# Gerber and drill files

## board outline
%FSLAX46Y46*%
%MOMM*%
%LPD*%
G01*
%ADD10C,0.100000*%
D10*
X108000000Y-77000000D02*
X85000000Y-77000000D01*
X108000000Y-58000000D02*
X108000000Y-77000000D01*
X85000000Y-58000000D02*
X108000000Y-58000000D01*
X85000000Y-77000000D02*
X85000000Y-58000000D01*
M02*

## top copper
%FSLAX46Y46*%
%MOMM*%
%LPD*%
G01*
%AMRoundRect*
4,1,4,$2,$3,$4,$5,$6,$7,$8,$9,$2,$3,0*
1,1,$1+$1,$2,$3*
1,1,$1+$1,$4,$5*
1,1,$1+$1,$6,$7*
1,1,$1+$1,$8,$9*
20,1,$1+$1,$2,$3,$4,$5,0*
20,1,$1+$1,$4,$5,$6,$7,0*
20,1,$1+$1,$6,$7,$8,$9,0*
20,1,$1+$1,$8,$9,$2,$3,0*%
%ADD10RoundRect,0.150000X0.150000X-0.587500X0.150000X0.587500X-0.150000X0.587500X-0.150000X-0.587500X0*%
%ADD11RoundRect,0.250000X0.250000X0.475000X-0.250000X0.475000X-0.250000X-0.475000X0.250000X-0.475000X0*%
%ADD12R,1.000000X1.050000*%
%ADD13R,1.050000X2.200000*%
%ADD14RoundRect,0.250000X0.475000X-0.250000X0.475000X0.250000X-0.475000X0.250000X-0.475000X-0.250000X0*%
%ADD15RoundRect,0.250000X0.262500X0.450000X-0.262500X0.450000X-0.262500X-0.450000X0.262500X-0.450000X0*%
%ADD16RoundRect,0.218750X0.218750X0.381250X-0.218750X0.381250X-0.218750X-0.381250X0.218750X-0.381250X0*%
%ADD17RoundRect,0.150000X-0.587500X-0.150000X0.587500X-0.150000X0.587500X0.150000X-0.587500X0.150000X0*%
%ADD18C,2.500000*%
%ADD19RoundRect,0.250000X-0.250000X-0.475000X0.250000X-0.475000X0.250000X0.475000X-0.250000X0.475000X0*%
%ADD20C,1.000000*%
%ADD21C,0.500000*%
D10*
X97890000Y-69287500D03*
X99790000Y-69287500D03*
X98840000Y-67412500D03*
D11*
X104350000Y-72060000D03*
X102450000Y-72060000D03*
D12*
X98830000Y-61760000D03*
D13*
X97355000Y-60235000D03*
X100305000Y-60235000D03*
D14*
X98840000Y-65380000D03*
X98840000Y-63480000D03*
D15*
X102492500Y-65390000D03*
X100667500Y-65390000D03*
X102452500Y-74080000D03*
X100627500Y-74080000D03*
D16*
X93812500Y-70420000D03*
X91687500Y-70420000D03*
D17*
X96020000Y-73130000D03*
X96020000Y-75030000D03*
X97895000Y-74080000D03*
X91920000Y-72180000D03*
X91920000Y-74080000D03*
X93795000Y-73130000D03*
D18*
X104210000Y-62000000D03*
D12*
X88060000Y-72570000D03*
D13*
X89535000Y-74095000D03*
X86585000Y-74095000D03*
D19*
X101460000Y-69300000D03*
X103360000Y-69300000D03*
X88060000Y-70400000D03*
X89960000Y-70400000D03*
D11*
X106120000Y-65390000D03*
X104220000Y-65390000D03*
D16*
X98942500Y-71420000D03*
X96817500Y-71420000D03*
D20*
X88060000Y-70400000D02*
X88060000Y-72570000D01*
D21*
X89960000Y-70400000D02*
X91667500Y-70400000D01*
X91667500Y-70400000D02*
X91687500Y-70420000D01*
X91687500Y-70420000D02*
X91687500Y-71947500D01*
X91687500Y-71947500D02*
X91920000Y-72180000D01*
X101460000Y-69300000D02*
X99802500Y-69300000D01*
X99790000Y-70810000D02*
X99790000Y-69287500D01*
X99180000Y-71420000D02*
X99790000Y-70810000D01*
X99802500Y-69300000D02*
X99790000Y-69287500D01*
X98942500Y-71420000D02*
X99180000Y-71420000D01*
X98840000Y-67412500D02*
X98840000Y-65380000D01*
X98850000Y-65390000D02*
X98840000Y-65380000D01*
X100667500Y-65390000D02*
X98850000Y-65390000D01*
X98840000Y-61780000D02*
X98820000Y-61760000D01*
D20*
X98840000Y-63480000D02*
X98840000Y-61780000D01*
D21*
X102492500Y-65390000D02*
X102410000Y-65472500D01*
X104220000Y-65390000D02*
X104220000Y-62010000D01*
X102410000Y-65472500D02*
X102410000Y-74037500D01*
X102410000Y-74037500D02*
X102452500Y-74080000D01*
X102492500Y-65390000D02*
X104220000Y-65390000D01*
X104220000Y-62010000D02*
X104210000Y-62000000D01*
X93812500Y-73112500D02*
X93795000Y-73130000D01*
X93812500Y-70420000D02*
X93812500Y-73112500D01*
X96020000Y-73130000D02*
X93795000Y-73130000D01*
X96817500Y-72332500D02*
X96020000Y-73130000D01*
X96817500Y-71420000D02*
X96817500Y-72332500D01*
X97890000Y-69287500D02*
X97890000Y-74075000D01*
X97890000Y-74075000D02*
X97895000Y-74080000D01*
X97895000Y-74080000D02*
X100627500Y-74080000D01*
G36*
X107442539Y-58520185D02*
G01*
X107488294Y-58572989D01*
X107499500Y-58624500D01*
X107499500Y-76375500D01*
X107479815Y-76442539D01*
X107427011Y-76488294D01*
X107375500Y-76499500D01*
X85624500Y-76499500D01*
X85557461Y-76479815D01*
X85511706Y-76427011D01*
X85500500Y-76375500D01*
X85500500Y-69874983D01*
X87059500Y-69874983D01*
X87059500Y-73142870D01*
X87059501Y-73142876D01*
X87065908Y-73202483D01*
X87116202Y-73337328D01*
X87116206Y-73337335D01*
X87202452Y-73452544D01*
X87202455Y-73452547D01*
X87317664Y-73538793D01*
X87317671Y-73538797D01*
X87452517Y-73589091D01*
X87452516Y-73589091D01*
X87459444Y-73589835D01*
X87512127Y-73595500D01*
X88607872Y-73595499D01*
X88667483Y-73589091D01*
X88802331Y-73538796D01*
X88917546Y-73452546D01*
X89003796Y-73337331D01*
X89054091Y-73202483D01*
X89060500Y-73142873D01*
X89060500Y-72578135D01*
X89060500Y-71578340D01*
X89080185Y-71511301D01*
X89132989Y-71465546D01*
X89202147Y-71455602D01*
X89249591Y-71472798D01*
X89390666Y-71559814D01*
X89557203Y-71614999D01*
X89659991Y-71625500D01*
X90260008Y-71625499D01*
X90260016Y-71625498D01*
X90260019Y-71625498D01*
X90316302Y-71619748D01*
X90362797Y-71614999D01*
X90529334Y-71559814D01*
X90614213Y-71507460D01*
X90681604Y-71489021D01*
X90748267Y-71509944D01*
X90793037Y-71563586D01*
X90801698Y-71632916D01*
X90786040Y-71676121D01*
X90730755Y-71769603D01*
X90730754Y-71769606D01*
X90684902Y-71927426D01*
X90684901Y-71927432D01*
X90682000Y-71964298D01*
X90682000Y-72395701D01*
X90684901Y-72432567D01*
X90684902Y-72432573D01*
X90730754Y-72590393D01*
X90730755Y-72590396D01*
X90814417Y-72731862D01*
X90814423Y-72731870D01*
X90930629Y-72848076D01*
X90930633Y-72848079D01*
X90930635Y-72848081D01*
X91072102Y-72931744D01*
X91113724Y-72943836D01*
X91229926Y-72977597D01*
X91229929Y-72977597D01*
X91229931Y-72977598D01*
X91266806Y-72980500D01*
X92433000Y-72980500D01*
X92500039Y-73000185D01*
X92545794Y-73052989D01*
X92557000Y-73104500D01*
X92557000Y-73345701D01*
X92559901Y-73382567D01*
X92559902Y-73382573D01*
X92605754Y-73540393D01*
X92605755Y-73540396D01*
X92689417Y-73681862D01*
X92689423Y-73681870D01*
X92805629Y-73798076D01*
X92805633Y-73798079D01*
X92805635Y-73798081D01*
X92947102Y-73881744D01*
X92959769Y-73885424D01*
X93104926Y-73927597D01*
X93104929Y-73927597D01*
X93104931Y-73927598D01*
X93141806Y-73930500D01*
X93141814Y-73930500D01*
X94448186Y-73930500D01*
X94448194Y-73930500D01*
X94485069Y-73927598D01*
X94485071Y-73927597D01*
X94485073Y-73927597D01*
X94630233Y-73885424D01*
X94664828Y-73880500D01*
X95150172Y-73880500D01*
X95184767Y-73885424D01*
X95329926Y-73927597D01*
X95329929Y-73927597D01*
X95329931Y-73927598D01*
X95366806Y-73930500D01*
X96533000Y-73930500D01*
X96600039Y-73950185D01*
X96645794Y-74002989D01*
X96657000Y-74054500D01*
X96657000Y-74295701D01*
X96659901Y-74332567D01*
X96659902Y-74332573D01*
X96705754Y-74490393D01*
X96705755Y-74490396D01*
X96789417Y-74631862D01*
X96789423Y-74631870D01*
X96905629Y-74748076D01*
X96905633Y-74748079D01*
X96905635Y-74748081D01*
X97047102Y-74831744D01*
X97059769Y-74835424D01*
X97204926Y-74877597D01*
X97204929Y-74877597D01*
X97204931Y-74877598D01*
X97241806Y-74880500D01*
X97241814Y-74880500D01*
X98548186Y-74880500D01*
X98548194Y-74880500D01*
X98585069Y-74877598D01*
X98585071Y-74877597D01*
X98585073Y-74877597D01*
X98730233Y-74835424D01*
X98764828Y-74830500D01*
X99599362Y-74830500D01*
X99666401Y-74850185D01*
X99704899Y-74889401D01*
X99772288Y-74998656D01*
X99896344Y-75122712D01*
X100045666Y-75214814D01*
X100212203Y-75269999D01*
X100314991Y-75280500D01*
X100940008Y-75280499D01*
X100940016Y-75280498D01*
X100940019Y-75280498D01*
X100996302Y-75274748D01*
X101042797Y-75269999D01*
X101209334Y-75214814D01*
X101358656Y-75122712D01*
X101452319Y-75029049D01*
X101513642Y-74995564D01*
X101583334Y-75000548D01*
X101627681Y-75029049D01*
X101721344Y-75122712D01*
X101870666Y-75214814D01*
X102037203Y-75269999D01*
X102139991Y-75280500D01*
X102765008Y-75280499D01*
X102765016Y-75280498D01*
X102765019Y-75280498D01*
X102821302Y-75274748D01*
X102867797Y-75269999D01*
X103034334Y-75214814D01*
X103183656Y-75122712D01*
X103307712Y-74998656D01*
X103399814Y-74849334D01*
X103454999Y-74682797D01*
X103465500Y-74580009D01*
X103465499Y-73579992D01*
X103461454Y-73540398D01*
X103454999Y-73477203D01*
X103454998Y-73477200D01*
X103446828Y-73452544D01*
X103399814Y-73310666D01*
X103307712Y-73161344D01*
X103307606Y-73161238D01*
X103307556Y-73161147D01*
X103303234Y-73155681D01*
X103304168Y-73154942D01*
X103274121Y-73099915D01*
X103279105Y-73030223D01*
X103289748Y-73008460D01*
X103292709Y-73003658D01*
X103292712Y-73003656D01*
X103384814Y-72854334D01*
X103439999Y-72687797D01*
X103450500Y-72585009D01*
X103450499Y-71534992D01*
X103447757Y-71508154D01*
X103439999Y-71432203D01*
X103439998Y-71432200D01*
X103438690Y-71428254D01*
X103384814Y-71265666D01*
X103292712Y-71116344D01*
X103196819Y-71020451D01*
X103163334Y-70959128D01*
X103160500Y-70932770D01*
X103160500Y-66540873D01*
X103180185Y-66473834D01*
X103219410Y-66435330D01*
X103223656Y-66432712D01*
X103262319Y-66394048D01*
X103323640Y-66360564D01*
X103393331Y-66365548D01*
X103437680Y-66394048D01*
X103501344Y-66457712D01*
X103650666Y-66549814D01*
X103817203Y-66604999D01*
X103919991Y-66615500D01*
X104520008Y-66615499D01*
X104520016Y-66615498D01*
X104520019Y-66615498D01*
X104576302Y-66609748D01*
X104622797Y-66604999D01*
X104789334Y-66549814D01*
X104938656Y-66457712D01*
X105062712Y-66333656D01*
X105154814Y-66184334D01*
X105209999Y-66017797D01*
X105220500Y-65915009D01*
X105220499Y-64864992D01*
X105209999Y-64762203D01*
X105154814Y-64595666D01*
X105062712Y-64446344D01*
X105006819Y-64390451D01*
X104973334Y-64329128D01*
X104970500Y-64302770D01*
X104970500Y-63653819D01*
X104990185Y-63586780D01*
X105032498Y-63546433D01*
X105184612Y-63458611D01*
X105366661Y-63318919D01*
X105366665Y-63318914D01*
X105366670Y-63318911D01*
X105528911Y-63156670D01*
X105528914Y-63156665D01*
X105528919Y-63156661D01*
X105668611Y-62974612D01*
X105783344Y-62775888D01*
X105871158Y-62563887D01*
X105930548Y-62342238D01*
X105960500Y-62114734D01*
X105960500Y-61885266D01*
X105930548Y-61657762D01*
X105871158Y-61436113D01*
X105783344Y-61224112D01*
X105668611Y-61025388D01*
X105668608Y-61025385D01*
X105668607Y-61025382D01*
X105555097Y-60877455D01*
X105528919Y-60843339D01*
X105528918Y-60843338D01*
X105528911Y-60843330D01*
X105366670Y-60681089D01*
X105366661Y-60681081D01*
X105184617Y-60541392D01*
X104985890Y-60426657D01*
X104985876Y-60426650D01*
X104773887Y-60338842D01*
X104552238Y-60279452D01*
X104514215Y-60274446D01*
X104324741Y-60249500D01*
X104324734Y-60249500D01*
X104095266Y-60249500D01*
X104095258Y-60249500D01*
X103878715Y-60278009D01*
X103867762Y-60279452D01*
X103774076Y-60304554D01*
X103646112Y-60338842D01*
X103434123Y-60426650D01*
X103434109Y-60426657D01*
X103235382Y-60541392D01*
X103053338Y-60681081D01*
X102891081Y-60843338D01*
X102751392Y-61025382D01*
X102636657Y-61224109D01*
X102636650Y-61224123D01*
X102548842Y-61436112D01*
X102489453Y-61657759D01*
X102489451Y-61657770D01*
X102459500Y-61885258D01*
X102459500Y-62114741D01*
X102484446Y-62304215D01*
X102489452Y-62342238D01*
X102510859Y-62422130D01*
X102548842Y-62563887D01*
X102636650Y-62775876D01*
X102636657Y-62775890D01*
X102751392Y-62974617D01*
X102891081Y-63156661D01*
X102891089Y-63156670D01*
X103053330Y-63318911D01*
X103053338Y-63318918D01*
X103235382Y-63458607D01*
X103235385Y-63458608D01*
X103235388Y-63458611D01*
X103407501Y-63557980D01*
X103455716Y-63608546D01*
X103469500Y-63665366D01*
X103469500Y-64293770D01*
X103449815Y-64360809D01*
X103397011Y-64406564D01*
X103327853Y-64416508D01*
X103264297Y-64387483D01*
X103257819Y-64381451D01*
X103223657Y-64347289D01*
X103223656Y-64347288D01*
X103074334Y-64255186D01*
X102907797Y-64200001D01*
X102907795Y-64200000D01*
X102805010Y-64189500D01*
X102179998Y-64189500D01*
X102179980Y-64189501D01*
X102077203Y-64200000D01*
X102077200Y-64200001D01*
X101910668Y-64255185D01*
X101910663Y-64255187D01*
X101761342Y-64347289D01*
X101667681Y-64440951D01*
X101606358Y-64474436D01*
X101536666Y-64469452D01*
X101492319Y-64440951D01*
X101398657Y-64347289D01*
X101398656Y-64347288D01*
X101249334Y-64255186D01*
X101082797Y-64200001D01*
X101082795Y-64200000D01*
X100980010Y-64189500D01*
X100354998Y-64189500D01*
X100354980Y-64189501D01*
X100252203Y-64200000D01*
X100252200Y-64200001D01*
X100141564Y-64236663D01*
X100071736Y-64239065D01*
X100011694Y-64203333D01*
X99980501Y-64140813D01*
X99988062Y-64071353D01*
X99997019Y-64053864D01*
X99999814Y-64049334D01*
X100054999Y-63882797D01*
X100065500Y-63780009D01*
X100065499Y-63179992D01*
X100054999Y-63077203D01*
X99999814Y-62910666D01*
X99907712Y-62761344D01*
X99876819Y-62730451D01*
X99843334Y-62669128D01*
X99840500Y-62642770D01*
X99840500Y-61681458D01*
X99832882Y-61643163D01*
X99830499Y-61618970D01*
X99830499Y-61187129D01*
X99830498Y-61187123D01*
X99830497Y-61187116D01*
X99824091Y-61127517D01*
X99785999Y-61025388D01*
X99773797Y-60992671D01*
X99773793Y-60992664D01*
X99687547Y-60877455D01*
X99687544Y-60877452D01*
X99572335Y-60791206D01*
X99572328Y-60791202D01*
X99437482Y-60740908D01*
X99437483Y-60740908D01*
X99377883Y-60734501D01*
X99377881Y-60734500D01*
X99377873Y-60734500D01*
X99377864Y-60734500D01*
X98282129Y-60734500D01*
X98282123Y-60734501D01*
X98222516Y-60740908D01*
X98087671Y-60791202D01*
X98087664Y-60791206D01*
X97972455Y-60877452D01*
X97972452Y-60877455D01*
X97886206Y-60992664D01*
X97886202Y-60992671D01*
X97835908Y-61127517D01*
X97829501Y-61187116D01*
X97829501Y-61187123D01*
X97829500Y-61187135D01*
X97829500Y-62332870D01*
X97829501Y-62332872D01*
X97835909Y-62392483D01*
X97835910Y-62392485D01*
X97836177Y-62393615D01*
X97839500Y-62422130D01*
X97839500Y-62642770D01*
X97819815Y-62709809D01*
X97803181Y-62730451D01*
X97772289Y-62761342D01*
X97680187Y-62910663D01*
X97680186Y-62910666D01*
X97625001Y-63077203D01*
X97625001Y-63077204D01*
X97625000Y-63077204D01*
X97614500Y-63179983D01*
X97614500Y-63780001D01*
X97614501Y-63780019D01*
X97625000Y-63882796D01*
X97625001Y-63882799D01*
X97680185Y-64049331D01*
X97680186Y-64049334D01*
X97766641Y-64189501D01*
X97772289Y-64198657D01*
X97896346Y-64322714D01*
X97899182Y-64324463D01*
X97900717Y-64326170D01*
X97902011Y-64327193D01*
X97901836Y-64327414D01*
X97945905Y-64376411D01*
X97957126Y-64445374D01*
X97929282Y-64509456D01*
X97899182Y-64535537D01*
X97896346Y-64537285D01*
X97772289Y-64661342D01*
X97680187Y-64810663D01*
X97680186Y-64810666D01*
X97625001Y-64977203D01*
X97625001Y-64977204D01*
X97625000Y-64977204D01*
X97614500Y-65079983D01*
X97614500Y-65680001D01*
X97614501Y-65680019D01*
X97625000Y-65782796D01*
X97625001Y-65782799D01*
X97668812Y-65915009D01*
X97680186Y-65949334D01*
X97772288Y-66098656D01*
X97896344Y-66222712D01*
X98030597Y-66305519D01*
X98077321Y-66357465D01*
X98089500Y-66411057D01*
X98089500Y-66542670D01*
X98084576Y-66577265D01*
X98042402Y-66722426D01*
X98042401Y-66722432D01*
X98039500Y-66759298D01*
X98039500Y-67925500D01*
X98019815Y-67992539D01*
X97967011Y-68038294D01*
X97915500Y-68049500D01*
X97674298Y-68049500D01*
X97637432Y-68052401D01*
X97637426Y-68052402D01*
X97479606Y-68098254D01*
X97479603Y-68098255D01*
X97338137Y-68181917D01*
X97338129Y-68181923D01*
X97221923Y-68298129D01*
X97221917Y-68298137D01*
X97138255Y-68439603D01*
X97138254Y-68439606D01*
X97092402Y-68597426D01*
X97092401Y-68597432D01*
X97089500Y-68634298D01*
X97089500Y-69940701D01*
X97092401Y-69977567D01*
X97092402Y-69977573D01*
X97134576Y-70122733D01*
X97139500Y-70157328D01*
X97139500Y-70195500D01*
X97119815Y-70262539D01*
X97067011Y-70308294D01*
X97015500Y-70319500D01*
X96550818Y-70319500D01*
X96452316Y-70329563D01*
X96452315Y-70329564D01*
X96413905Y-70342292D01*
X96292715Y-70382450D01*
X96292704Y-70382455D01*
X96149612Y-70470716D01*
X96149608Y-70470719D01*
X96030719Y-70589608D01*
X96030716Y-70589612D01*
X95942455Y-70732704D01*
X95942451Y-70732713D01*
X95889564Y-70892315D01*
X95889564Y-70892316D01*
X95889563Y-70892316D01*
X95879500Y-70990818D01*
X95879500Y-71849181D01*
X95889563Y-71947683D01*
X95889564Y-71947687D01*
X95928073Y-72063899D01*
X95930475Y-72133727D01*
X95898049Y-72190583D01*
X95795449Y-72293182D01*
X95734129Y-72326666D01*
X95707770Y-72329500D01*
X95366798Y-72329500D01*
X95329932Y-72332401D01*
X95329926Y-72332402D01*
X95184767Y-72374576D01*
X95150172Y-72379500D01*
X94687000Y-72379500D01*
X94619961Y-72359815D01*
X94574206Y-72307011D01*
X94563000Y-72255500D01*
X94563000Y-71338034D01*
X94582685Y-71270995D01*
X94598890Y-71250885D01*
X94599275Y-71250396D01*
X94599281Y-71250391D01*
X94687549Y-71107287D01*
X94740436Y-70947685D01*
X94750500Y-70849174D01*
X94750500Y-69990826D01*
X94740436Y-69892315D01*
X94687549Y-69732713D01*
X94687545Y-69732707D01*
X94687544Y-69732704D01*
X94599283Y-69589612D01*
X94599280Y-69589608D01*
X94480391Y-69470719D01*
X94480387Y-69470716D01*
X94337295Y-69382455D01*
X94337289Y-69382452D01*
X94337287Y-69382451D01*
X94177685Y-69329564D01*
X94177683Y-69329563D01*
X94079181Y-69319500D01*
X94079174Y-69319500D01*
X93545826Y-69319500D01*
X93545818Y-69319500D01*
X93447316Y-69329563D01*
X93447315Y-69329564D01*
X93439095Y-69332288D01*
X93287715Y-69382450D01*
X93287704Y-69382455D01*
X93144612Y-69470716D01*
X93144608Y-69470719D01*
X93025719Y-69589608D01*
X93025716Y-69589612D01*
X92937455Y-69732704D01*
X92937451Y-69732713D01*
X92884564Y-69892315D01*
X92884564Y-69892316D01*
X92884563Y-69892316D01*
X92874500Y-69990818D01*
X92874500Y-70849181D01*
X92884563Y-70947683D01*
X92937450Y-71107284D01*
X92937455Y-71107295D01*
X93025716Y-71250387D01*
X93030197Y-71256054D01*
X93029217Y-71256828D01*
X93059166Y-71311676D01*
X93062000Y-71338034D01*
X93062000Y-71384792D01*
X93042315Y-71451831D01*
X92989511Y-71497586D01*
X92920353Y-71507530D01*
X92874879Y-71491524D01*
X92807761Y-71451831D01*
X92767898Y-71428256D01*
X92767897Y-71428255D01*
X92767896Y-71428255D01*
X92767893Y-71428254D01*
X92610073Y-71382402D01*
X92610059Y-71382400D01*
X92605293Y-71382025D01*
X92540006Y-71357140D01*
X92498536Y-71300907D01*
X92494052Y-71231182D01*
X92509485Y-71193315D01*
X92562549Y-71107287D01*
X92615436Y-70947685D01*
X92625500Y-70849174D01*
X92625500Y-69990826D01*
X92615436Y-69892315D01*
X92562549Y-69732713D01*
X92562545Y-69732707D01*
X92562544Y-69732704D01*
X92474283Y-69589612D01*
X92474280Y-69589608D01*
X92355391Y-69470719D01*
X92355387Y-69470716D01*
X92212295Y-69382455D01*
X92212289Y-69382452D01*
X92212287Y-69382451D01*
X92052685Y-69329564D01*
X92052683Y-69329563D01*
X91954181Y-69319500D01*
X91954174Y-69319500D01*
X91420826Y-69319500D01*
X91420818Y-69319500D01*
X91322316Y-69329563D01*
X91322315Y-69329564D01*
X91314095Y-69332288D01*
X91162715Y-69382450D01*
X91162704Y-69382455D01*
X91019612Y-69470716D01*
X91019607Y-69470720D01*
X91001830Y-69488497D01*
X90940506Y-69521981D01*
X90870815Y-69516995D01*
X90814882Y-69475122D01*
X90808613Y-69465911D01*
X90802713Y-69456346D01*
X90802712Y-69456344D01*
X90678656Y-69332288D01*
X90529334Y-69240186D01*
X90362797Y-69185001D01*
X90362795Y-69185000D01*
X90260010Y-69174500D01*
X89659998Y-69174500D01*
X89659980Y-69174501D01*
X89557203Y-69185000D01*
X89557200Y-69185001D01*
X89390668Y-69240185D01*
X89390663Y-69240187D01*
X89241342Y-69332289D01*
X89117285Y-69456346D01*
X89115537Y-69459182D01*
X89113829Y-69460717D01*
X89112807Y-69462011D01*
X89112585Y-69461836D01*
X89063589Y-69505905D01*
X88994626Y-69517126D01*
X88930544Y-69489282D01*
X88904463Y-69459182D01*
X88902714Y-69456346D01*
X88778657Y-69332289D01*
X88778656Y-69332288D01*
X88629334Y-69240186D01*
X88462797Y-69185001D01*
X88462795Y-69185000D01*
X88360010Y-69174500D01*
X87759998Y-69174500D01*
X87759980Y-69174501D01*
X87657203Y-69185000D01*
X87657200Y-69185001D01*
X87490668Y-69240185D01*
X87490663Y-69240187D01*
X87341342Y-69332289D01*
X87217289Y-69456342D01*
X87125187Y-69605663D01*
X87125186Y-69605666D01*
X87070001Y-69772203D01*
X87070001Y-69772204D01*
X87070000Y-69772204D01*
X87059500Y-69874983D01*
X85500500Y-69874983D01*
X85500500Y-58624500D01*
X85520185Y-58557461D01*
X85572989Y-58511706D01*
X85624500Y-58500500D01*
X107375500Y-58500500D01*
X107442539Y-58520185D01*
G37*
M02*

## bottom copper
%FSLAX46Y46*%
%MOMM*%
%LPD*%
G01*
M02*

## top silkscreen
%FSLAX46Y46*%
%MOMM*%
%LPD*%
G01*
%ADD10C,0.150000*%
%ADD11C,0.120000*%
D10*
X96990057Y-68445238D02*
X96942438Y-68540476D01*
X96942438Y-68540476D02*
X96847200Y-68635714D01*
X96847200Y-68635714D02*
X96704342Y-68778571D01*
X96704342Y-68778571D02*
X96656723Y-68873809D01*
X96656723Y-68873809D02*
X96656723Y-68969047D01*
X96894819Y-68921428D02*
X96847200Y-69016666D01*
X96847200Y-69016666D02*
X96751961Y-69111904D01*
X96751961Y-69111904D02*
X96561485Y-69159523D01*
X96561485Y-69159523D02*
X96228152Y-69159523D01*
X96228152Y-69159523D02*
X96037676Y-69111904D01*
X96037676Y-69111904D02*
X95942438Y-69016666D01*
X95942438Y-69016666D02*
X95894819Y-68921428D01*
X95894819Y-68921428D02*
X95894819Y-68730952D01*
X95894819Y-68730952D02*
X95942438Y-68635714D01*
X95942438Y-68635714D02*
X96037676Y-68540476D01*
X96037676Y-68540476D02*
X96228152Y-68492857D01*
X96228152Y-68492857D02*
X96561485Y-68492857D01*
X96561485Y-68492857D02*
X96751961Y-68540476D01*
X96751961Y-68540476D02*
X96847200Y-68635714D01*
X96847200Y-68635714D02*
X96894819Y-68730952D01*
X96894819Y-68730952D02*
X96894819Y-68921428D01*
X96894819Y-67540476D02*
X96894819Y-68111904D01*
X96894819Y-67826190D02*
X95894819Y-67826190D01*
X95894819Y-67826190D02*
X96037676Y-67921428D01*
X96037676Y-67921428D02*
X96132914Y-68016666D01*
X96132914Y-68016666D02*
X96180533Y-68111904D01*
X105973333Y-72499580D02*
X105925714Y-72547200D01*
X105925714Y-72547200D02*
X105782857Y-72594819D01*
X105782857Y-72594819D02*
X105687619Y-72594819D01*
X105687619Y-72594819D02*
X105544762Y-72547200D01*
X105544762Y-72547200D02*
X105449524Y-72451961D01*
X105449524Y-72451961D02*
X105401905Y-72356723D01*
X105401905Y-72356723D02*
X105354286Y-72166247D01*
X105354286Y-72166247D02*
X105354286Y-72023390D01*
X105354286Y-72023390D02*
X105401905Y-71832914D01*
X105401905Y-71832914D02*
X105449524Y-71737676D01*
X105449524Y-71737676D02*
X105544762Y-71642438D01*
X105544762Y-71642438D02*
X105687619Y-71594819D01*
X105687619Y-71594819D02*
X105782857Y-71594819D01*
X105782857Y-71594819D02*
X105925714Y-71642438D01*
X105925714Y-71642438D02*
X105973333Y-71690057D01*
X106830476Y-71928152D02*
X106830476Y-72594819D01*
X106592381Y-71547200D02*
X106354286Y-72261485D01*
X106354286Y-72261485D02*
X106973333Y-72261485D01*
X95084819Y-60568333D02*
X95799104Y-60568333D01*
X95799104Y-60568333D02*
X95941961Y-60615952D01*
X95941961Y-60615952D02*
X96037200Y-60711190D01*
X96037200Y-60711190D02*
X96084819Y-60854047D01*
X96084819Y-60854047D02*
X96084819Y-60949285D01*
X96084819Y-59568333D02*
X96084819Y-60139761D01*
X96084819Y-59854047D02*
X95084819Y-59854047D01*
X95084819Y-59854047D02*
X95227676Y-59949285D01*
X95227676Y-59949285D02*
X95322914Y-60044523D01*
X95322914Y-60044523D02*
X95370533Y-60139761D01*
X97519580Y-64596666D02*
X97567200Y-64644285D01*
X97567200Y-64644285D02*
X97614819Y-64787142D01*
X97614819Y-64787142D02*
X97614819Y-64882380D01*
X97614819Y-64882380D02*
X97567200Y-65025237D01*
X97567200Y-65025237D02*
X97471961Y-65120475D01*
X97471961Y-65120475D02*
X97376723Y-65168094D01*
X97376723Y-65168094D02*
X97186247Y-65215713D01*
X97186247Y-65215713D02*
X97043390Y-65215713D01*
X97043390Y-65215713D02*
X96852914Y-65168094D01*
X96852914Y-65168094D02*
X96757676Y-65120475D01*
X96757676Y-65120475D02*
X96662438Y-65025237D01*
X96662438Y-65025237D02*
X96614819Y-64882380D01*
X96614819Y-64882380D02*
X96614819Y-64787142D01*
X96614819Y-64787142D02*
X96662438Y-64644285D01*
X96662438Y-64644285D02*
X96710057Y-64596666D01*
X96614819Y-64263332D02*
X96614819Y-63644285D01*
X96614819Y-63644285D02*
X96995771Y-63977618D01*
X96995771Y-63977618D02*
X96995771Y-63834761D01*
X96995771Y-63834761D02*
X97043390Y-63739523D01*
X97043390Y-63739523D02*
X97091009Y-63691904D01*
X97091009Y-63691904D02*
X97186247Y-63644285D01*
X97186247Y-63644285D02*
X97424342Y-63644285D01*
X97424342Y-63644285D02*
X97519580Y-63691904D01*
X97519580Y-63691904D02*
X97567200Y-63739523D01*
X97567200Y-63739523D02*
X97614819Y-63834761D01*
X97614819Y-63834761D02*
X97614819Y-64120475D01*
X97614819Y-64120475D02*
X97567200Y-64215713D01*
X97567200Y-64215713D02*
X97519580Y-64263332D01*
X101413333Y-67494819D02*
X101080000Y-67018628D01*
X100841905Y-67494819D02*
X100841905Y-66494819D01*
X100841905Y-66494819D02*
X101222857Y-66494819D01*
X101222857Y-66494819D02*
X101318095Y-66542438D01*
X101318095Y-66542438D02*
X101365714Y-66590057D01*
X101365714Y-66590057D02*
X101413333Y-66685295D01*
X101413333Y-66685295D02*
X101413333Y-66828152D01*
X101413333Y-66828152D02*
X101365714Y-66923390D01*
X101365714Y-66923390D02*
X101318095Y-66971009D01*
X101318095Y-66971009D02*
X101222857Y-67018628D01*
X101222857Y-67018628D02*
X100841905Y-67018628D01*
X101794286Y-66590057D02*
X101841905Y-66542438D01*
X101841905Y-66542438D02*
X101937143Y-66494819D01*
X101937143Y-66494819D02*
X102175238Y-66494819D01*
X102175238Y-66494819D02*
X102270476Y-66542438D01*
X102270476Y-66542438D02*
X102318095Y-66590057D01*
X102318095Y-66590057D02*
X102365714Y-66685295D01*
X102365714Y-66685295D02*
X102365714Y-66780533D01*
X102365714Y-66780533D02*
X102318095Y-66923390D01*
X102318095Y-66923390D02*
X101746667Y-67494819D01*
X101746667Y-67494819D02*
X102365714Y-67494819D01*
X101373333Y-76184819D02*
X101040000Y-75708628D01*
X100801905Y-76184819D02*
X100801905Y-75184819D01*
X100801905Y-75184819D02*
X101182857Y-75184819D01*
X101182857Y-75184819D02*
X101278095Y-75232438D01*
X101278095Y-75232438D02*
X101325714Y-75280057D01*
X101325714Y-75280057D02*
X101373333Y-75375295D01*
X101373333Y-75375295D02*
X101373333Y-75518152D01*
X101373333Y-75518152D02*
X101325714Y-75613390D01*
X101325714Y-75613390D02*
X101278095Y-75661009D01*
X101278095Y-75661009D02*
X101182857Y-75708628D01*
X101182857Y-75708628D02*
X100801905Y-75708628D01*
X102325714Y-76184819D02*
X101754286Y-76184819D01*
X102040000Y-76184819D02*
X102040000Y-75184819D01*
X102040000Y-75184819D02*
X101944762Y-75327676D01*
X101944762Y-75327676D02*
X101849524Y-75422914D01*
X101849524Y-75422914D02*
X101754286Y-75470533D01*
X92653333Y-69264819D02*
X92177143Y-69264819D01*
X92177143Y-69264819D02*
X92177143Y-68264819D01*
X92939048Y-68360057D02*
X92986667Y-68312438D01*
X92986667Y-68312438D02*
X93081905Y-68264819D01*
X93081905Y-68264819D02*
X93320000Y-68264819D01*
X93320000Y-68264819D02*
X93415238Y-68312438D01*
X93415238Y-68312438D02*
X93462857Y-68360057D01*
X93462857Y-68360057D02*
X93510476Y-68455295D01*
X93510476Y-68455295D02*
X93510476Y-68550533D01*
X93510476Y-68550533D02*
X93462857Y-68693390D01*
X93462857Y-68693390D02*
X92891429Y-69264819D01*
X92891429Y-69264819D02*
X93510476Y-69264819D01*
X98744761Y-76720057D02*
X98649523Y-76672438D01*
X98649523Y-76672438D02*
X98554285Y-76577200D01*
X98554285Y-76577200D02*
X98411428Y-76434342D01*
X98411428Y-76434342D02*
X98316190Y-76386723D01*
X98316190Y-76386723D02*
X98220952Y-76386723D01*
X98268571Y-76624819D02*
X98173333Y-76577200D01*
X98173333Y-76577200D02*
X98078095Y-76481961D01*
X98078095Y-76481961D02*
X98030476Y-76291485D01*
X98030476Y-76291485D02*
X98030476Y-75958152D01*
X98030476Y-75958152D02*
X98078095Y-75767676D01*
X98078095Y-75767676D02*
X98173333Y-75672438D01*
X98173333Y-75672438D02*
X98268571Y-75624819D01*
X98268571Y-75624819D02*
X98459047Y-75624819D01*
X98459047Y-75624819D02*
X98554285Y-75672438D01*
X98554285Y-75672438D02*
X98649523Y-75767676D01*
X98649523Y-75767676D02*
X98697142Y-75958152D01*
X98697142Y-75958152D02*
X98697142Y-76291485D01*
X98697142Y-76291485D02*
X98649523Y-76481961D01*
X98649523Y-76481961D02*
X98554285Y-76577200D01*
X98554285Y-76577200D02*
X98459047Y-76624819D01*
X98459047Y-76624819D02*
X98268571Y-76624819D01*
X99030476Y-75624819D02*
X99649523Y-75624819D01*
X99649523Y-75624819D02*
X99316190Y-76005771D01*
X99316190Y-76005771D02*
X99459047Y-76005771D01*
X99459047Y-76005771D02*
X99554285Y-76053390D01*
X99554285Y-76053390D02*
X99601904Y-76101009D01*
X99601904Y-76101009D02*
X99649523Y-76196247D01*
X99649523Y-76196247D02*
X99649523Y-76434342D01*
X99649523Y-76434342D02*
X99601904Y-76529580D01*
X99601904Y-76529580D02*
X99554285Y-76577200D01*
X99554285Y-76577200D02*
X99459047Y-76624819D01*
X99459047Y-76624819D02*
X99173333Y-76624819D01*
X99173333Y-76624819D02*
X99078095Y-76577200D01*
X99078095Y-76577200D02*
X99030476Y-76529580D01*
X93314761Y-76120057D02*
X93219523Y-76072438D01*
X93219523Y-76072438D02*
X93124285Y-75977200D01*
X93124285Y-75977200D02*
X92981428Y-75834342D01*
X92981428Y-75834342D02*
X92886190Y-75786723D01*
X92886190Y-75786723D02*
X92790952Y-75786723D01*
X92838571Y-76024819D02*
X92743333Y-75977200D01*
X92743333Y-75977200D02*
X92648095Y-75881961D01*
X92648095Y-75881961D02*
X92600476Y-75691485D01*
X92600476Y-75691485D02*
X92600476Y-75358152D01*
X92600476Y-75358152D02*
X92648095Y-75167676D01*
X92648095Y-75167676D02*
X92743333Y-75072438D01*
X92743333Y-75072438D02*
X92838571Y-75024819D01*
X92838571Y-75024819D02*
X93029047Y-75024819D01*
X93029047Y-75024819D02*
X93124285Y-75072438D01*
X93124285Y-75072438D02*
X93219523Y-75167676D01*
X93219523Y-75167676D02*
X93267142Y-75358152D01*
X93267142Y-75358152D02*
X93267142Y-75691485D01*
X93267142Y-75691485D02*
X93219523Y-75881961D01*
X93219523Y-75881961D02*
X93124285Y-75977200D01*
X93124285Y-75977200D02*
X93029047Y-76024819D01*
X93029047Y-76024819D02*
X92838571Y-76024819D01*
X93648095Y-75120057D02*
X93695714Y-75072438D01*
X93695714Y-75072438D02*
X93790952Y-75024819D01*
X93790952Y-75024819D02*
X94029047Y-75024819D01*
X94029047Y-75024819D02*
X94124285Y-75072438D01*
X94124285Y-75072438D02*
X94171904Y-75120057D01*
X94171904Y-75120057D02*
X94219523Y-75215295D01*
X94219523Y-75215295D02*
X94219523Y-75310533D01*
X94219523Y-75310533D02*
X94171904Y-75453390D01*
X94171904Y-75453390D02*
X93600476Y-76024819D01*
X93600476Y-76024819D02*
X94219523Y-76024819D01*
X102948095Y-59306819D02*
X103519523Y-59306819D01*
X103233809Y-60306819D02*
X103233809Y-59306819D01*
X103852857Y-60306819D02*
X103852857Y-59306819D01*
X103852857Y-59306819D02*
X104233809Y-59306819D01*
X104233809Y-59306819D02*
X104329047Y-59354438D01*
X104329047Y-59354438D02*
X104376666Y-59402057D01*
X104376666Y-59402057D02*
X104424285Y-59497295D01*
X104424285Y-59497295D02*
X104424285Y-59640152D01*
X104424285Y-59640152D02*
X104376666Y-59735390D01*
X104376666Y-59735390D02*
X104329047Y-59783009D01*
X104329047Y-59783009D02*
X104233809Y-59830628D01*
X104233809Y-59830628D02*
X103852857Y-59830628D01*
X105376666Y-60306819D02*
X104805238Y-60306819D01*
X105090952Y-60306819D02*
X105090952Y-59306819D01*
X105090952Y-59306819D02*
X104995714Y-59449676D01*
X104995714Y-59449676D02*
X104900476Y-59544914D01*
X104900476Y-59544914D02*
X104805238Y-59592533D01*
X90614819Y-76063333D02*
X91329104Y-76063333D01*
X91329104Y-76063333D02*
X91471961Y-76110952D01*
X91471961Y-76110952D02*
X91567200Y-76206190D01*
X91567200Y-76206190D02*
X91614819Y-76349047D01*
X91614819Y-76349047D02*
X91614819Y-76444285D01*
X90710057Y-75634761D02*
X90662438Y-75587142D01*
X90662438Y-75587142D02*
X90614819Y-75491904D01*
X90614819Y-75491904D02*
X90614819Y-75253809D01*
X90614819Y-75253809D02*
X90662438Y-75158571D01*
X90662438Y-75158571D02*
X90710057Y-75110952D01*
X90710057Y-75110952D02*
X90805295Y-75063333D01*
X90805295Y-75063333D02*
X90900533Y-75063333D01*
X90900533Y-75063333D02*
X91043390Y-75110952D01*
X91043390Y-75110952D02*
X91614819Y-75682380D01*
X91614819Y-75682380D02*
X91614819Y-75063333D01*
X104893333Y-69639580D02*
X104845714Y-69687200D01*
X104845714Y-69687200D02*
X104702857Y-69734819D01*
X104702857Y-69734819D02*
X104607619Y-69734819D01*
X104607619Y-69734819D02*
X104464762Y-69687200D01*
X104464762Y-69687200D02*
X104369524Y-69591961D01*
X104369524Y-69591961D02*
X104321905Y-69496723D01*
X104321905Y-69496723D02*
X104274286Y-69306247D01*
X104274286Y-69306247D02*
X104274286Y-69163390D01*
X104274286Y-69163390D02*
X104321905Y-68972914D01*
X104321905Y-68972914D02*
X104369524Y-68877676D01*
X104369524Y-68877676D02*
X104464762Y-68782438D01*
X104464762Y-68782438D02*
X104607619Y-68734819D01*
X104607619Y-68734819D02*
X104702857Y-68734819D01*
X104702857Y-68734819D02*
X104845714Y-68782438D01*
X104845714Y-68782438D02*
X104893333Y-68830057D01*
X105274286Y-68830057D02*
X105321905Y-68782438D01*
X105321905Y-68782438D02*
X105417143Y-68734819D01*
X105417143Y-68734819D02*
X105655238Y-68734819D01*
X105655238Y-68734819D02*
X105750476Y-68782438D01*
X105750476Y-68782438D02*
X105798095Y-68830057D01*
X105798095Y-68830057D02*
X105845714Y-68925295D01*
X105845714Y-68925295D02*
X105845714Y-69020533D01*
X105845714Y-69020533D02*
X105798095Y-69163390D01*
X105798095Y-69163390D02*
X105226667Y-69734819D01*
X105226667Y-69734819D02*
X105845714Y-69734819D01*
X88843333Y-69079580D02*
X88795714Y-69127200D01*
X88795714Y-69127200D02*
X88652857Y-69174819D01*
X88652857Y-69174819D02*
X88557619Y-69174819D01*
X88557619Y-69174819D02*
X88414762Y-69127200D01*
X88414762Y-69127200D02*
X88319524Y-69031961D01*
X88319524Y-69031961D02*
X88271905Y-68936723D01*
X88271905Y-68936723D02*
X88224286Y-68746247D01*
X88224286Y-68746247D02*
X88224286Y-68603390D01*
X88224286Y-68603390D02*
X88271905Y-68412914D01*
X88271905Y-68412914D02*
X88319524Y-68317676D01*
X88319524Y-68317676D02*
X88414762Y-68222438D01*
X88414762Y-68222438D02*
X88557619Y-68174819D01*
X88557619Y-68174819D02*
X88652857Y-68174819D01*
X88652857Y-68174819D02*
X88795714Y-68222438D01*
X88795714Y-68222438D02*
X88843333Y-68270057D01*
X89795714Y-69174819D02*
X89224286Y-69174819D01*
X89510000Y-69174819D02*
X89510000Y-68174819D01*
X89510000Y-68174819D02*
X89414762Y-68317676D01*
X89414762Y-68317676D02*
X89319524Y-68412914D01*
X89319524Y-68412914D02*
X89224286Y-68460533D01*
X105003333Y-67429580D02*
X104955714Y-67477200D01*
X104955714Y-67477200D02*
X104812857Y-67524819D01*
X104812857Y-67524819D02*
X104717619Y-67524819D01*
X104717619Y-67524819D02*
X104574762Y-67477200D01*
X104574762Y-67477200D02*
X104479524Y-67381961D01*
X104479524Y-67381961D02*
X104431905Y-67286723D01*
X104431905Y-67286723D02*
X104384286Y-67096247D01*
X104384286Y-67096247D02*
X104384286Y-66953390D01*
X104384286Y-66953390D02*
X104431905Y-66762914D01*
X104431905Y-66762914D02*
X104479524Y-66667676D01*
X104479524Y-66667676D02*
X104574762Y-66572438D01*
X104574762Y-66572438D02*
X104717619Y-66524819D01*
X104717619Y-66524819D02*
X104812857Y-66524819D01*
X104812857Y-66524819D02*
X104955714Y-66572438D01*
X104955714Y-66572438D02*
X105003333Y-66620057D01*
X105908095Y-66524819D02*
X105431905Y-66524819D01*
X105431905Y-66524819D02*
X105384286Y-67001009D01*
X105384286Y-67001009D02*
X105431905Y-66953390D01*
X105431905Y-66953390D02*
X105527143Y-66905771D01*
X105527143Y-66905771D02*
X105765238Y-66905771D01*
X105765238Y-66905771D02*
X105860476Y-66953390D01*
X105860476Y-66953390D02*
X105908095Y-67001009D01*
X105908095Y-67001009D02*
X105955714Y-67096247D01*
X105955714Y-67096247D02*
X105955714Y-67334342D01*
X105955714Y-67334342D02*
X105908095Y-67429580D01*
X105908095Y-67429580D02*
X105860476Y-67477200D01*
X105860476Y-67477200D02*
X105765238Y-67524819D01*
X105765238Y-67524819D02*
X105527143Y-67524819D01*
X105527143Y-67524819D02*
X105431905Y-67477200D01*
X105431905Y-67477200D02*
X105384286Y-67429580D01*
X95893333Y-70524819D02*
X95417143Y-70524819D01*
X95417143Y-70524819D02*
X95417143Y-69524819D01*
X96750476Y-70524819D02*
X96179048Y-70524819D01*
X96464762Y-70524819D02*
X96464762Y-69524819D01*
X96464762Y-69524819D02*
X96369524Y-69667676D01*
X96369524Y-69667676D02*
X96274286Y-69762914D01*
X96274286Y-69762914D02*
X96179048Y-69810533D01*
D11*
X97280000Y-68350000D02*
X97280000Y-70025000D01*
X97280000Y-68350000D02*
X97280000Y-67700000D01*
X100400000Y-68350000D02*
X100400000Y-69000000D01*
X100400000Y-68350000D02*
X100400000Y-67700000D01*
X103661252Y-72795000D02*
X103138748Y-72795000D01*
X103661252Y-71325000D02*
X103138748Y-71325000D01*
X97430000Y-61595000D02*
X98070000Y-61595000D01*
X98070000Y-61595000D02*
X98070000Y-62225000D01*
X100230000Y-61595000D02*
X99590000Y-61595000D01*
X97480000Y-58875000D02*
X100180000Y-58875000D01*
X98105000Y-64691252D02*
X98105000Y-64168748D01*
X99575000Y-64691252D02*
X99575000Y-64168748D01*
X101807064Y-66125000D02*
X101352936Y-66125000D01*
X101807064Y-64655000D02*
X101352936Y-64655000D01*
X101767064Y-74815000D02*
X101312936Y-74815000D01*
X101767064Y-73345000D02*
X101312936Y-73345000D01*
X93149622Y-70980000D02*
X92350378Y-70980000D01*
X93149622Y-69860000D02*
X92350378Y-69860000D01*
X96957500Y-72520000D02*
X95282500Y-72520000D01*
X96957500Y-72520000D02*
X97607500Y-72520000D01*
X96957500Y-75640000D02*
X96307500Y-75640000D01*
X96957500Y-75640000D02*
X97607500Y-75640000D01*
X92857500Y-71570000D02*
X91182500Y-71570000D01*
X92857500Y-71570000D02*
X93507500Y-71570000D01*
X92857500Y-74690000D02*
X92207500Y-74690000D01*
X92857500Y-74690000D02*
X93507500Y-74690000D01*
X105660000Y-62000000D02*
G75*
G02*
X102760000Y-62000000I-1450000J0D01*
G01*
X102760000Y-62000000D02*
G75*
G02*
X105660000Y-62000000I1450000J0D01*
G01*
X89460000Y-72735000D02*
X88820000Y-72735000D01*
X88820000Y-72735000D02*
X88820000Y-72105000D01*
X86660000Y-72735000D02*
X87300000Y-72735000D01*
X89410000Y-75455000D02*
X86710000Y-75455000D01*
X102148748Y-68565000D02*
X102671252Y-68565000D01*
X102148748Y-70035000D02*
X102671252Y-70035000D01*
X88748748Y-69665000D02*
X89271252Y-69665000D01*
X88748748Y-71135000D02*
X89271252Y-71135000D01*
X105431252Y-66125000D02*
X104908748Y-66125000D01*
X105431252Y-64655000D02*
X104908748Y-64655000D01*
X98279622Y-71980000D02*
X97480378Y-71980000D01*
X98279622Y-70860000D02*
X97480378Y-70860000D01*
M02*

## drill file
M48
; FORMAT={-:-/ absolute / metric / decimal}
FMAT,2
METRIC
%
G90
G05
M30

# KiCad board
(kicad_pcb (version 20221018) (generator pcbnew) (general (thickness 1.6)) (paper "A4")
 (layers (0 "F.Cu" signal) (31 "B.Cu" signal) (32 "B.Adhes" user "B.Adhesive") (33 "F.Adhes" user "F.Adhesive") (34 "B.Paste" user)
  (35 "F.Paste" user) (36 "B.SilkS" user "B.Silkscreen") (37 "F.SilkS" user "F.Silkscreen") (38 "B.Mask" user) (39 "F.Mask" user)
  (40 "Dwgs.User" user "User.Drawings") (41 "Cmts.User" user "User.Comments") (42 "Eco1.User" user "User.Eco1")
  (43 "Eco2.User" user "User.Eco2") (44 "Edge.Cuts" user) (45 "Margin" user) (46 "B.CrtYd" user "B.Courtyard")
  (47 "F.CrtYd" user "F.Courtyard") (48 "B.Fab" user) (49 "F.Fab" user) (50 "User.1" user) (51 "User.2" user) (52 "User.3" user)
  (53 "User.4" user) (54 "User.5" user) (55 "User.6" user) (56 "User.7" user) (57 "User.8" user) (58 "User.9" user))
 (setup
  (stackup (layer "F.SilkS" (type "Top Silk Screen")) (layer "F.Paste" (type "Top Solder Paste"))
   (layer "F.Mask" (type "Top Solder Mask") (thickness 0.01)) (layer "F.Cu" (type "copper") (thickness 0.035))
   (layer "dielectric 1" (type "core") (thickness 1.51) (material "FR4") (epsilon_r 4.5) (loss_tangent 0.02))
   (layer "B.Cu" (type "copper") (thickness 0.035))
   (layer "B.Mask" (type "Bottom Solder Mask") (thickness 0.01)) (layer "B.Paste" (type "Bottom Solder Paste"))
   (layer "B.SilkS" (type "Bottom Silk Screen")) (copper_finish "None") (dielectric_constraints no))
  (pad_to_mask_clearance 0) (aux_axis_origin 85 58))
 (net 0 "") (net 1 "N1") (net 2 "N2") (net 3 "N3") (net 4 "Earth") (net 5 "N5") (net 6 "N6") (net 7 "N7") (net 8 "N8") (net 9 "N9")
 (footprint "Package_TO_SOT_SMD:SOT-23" (layer "F.Cu") (at 98.84 68.35 90)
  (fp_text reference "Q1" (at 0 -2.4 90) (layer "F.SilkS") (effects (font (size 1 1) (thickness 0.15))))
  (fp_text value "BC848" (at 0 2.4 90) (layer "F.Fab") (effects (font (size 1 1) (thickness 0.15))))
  (fp_line (start 0 -1.56) (end -1.675 -1.56) (stroke (width 0.12) (type solid)) (layer "F.SilkS"))
  (fp_line (start 0 -1.56) (end 0.65 -1.56) (stroke (width 0.12) (type solid)) (layer "F.SilkS"))
  (fp_line (start 0 1.56) (end -0.65 1.56) (stroke (width 0.12) (type solid)) (layer "F.SilkS"))
  (fp_line (start 0 1.56) (end 0.65 1.56) (stroke (width 0.12) (type solid)) (layer "F.SilkS"))
  (pad "1" smd roundrect (at -0.9375 -0.95 90) (size 1.475 0.6) (layers "F.Cu" "F.Paste" "F.Mask") (roundrect_rratio 0.25) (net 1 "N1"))
  (pad "2" smd roundrect (at -0.9375 0.95 90) (size 1.475 0.6) (layers "F.Cu" "F.Paste" "F.Mask") (roundrect_rratio 0.25) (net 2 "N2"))
  (pad "3" smd roundrect (at 0.9375 0 90) (size 1.475 0.6) (layers "F.Cu" "F.Paste" "F.Mask") (roundrect_rratio 0.25) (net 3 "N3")))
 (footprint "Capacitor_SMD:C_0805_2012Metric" (layer "F.Cu") (at 103.4 72.06 180)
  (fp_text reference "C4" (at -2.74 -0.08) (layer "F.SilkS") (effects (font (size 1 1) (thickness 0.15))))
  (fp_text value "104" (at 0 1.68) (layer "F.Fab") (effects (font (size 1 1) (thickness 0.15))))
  (fp_line (start -0.261252 -0.735) (end 0.261252 -0.735) (stroke (width 0.12) (type solid)) (layer "F.SilkS"))
  (fp_line (start -0.261252 0.735) (end 0.261252 0.735) (stroke (width 0.12) (type solid)) (layer "F.SilkS"))
  (pad "1" smd roundrect (at -0.95 0 180) (size 1 1.45) (layers "F.Cu" "F.Paste" "F.Mask") (roundrect_rratio 0.25) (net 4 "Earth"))
  (pad "2" smd roundrect (at 0.95 0 180) (size 1 1.45) (layers "F.Cu" "F.Paste" "F.Mask") (roundrect_rratio 0.25) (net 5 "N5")))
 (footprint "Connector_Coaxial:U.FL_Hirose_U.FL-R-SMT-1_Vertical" (layer "F.Cu") (at 98.83 60.71 90)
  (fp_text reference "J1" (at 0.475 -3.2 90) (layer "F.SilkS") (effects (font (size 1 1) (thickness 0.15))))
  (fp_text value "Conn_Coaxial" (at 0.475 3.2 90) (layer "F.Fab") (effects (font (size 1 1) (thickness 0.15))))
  (fp_line (start -0.885 -1.4) (end -0.885 -0.76) (stroke (width 0.12) (type solid)) (layer "F.SilkS"))
  (fp_line (start -0.885 -0.76) (end -1.515 -0.76) (stroke (width 0.12) (type solid)) (layer "F.SilkS"))
  (fp_line (start -0.885 1.4) (end -0.885 0.76) (stroke (width 0.12) (type solid)) (layer "F.SilkS"))
  (fp_line (start 1.835 -1.35) (end 1.835 1.35) (stroke (width 0.12) (type solid)) (layer "F.SilkS"))
  (pad "1" smd rect (at -1.05 0 90) (size 1.05 1) (layers "F.Cu" "F.Paste" "F.Mask") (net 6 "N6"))
  (pad "2" smd rect (at 0.475 -1.475 90) (size 2.2 1.05) (layers "F.Cu" "F.Paste" "F.Mask") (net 4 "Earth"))
  (pad "2" smd rect (at 0.475 1.475 90) (size 2.2 1.05) (layers "F.Cu" "F.Paste" "F.Mask") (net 4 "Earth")))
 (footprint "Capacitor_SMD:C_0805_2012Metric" (layer "F.Cu") (at 98.84 64.43 90)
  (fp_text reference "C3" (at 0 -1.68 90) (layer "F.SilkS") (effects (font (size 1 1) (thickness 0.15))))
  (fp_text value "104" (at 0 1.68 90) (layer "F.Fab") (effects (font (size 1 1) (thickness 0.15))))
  (fp_line (start -0.261252 -0.735) (end 0.261252 -0.735) (stroke (width 0.12) (type solid)) (layer "F.SilkS"))
  (fp_line (start -0.261252 0.735) (end 0.261252 0.735) (stroke (width 0.12) (type solid)) (layer "F.SilkS"))
  (pad "1" smd roundrect (at -0.95 0 90) (size 1 1.45) (layers "F.Cu" "F.Paste" "F.Mask") (roundrect_rratio 0.25) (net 3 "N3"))
  (pad "2" smd roundrect (at 0.95 0 90) (size 1 1.45) (layers "F.Cu" "F.Paste" "F.Mask") (roundrect_rratio 0.25) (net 6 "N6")))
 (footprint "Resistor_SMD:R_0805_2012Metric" (layer "F.Cu") (at 101.58 65.39 180)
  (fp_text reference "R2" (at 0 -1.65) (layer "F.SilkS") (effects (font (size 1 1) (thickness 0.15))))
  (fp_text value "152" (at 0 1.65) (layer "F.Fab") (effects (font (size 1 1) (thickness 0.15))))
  (fp_line (start -0.227064 -0.735) (end 0.227064 -0.735) (stroke (width 0.12) (type solid)) (layer "F.SilkS"))
  (fp_line (start -0.227064 0.735) (end 0.227064 0.735) (stroke (width 0.12) (type solid)) (layer "F.SilkS"))
  (pad "1" smd roundrect (at -0.9125 0 180) (size 1.025 1.4) (layers "F.Cu" "F.Paste" "F.Mask") (roundrect_rratio 0.243902439) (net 5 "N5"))
  (pad "2" smd roundrect (at 0.9125 0 180) (size 1.025 1.4) (layers "F.Cu" "F.Paste" "F.Mask") (roundrect_rratio 0.243902439) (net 3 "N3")))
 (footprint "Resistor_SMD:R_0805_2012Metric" (layer "F.Cu") (at 101.54 74.08 180)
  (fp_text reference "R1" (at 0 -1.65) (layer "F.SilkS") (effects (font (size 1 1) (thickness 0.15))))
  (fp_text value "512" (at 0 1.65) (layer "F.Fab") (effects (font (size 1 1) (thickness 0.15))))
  (fp_line (start -0.227064 -0.735) (end 0.227064 -0.735) (stroke (width 0.12) (type solid)) (layer "F.SilkS"))
  (fp_line (start -0.227064 0.735) (end 0.227064 0.735) (stroke (width 0.12) (type solid)) (layer "F.SilkS"))
  (pad "1" smd roundrect (at -0.9125 0 180) (size 1.025 1.4) (layers "F.Cu" "F.Paste" "F.Mask") (roundrect_rratio 0.243902439) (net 5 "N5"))
  (pad "2" smd roundrect (at 0.9125 0 180) (size 1.025 1.4) (layers "F.Cu" "F.Paste" "F.Mask") (roundrect_rratio 0.243902439) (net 1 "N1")))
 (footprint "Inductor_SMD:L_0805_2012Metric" (layer "F.Cu") (at 92.75 70.42 180)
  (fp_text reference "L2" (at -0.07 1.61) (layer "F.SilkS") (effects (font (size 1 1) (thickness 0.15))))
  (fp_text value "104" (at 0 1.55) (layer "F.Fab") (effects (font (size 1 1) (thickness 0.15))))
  (fp_line (start -0.399622 -0.56) (end 0.399622 -0.56) (stroke (width 0.12) (type solid)) (layer "F.SilkS"))
  (fp_line (start -0.399622 0.56) (end 0.399622 0.56) (stroke (width 0.12) (type solid)) (layer "F.SilkS"))
  (pad "1" smd roundrect (at -1.0625 0 180) (size 0.875 1.2) (layers "F.Cu" "F.Paste" "F.Mask") (roundrect_rratio 0.25) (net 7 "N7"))
  (pad "2" smd roundrect (at 1.0625 0 180) (size 0.875 1.2) (layers "F.Cu" "F.Paste" "F.Mask") (roundrect_rratio 0.25) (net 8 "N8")))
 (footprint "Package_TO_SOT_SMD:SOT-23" (layer "F.Cu") (at 96.9575 74.08)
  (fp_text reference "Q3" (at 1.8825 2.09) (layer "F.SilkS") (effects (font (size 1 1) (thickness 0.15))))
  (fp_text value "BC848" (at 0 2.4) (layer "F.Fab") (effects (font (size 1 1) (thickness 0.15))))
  (fp_line (start 0 -1.56) (end -1.675 -1.56) (stroke (width 0.12) (type solid)) (layer "F.SilkS"))
  (fp_line (start 0 -1.56) (end 0.65 -1.56) (stroke (width 0.12) (type solid)) (layer "F.SilkS"))
  (fp_line (start 0 1.56) (end -0.65 1.56) (stroke (width 0.12) (type solid)) (layer "F.SilkS"))
  (fp_line (start 0 1.56) (end 0.65 1.56) (stroke (width 0.12) (type solid)) (layer "F.SilkS"))
  (pad "1" smd roundrect (at -0.9375 -0.95) (size 1.475 0.6) (layers "F.Cu" "F.Paste" "F.Mask") (roundrect_rratio 0.25) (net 7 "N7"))
  (pad "2" smd roundrect (at -0.9375 0.95) (size 1.475 0.6) (layers "F.Cu" "F.Paste" "F.Mask") (roundrect_rratio 0.25) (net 4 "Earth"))
  (pad "3" smd roundrect (at 0.9375 0) (size 1.475 0.6) (layers "F.Cu" "F.Paste" "F.Mask") (roundrect_rratio 0.25) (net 1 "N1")))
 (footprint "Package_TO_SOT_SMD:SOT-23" (layer "F.Cu") (at 92.8575 73.13)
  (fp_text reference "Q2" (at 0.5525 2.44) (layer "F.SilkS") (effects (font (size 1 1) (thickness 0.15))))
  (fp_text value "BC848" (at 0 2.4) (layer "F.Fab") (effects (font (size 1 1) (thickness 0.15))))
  (fp_line (start 0 -1.56) (end -1.675 -1.56) (stroke (width 0.12) (type solid)) (layer "F.SilkS"))
  (fp_line (start 0 -1.56) (end 0.65 -1.56) (stroke (width 0.12) (type solid)) (layer "F.SilkS"))
  (fp_line (start 0 1.56) (end -0.65 1.56) (stroke (width 0.12) (type solid)) (layer "F.SilkS"))
  (fp_line (start 0 1.56) (end 0.65 1.56) (stroke (width 0.12) (type solid)) (layer "F.SilkS"))
  (pad "1" smd roundrect (at -0.9375 -0.95) (size 1.475 0.6) (layers "F.Cu" "F.Paste" "F.Mask") (roundrect_rratio 0.25) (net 8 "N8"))
  (pad "2" smd roundrect (at -0.9375 0.95) (size 1.475 0.6) (layers "F.Cu" "F.Paste" "F.Mask") (roundrect_rratio 0.25) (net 4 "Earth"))
  (pad "3" smd roundrect (at 0.9375 0) (size 1.475 0.6) (layers "F.Cu" "F.Paste" "F.Mask") (roundrect_rratio 0.25) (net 7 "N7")))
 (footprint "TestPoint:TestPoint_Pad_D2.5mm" (layer "F.Cu") (at 104.21 62)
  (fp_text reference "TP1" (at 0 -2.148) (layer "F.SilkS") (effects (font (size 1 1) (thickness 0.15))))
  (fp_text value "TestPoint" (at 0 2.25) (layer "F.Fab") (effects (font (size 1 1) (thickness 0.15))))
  (fp_circle (center 0 0) (end 0 1.45) (stroke (width 0.12) (type solid)) (fill none) (layer "F.SilkS"))
  (pad "1" smd circle (at 0 0) (size 2.5 2.5) (layers "F.Cu" "F.Mask") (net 5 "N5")))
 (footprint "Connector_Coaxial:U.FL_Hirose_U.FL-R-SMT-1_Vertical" (layer "F.Cu") (at 88.06 73.62 -90)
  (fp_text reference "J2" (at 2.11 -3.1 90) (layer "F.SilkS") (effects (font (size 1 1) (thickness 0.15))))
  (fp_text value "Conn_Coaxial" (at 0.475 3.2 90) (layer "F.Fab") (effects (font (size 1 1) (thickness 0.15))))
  (fp_line (start -0.885 -1.4) (end -0.885 -0.76) (stroke (width 0.12) (type solid)) (layer "F.SilkS"))
  (fp_line (start -0.885 -0.76) (end -1.515 -0.76) (stroke (width 0.12) (type solid)) (layer "F.SilkS"))
  (fp_line (start -0.885 1.4) (end -0.885 0.76) (stroke (width 0.12) (type solid)) (layer "F.SilkS"))
  (fp_line (start 1.835 -1.35) (end 1.835 1.35) (stroke (width 0.12) (type solid)) (layer "F.SilkS"))
  (pad "1" smd rect (at -1.05 0 270) (size 1.05 1) (layers "F.Cu" "F.Paste" "F.Mask") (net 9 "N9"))
  (pad "2" smd rect (at 0.475 -1.475 270) (size 2.2 1.05) (layers "F.Cu" "F.Paste" "F.Mask") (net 4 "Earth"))
  (pad "2" smd rect (at 0.475 1.475 270) (size 2.2 1.05) (layers "F.Cu" "F.Paste" "F.Mask") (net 4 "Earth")))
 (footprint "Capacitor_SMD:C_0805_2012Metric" (layer "F.Cu") (at 102.41 69.3)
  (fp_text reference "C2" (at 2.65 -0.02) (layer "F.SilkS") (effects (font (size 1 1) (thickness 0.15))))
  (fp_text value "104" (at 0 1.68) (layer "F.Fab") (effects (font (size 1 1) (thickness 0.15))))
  (fp_line (start -0.261252 -0.735) (end 0.261252 -0.735) (stroke (width 0.12) (type solid)) (layer "F.SilkS"))
  (fp_line (start -0.261252 0.735) (end 0.261252 0.735) (stroke (width 0.12) (type solid)) (layer "F.SilkS"))
  (pad "1" smd roundrect (at -0.95 0) (size 1 1.45) (layers "F.Cu" "F.Paste" "F.Mask") (roundrect_rratio 0.25) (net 2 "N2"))
  (pad "2" smd roundrect (at 0.95 0) (size 1 1.45) (layers "F.Cu" "F.Paste" "F.Mask") (roundrect_rratio 0.25) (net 4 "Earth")))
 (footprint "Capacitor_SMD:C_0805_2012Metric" (layer "F.Cu") (at 89.01 70.4)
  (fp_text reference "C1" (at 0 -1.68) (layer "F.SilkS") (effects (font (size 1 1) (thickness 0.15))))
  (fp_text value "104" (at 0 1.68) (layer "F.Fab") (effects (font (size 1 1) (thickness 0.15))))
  (fp_line (start -0.261252 -0.735) (end 0.261252 -0.735) (stroke (width 0.12) (type solid)) (layer "F.SilkS"))
  (fp_line (start -0.261252 0.735) (end 0.261252 0.735) (stroke (width 0.12) (type solid)) (layer "F.SilkS"))
  (pad "1" smd roundrect (at -0.95 0) (size 1 1.45) (layers "F.Cu" "F.Paste" "F.Mask") (roundrect_rratio 0.25) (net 9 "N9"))
  (pad "2" smd roundrect (at 0.95 0) (size 1 1.45) (layers "F.Cu" "F.Paste" "F.Mask") (roundrect_rratio 0.25) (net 8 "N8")))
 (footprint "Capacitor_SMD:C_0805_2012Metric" (layer "F.Cu") (at 105.17 65.39 180)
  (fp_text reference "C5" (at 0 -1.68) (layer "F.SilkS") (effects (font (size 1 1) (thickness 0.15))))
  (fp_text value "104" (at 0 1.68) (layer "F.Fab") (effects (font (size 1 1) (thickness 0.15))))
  (fp_line (start -0.261252 -0.735) (end 0.261252 -0.735) (stroke (width 0.12) (type solid)) (layer "F.SilkS"))
  (fp_line (start -0.261252 0.735) (end 0.261252 0.735) (stroke (width 0.12) (type solid)) (layer "F.SilkS"))
  (pad "1" smd roundrect (at -0.95 0 180) (size 1 1.45) (layers "F.Cu" "F.Paste" "F.Mask") (roundrect_rratio 0.25) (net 4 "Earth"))
  (pad "2" smd roundrect (at 0.95 0 180) (size 1 1.45) (layers "F.Cu" "F.Paste" "F.Mask") (roundrect_rratio 0.25) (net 5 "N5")))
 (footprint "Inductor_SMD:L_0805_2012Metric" (layer "F.Cu") (at 97.88 71.42 180)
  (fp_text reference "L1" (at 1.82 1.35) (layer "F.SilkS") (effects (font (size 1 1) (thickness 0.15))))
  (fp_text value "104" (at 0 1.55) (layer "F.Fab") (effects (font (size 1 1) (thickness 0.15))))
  (fp_line (start -0.399622 -0.56) (end 0.399622 -0.56) (stroke (width 0.12) (type solid)) (layer "F.SilkS"))
  (fp_line (start -0.399622 0.56) (end 0.399622 0.56) (stroke (width 0.12) (type solid)) (layer "F.SilkS"))
  (pad "1" smd roundrect (at -1.0625 0 180) (size 0.875 1.2) (layers "F.Cu" "F.Paste" "F.Mask") (roundrect_rratio 0.25) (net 2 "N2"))
  (pad "2" smd roundrect (at 1.0625 0 180) (size 0.875 1.2) (layers "F.Cu" "F.Paste" "F.Mask") (roundrect_rratio 0.25) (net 7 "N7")))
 (gr_line (start 108 77) (end 85 77) (stroke (width 0.1) (type default)) (layer "Edge.Cuts"))
 (gr_line (start 108 58) (end 108 77) (stroke (width 0.1) (type default)) (layer "Edge.Cuts"))
 (gr_line (start 85 58) (end 108 58) (stroke (width 0.1) (type default)) (layer "Edge.Cuts"))
 (gr_line (start 85 77) (end 85 58) (stroke (width 0.1) (type default)) (layer "Edge.Cuts"))
 (segment (start 88.06 70.4) (end 88.06 72.57) (width 1) (layer "F.Cu") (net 9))
 (segment (start 89.96 70.4) (end 91.6675 70.4) (width 0.5) (layer "F.Cu") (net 8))
 (segment (start 91.6675 70.4) (end 91.6875 70.42) (width 0.5) (layer "F.Cu") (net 8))
 (segment (start 91.6875 70.42) (end 91.6875 71.9475) (width 0.5) (layer "F.Cu") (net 8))
 (segment (start 91.6875 71.9475) (end 91.92 72.18) (width 0.5) (layer "F.Cu") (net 8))
 (segment (start 101.46 69.3) (end 99.8025 69.3) (width 0.5) (layer "F.Cu") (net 2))
 (segment (start 99.79 70.81) (end 99.79 69.2875) (width 0.5) (layer "F.Cu") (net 2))
 (segment (start 99.18 71.42) (end 99.79 70.81) (width 0.5) (layer "F.Cu") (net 2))
 (segment (start 99.8025 69.3) (end 99.79 69.2875) (width 0.5) (layer "F.Cu") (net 2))
 (segment (start 98.9425 71.42) (end 99.18 71.42) (width 0.5) (layer "F.Cu") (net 2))
 (segment (start 98.84 67.4125) (end 98.84 65.38) (width 0.5) (layer "F.Cu") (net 3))
 (segment (start 98.85 65.39) (end 98.84 65.38) (width 0.5) (layer "F.Cu") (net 3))
 (segment (start 100.6675 65.39) (end 98.85 65.39) (width 0.5) (layer "F.Cu") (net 3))
 (segment (start 98.84 61.78) (end 98.82 61.76) (width 0.5) (layer "F.Cu") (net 6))
 (segment (start 98.84 63.48) (end 98.84 61.78) (width 1) (layer "F.Cu") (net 6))
 (segment (start 102.4925 65.39) (end 102.41 65.4725) (width 0.5) (layer "F.Cu") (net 5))
 (segment (start 104.22 65.39) (end 104.22 62.01) (width 0.5) (layer "F.Cu") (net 5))
 (segment (start 102.41 65.4725) (end 102.41 74.0375) (width 0.5) (layer "F.Cu") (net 5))
 (segment (start 102.41 74.0375) (end 102.4525 74.08) (width 0.5) (layer "F.Cu") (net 5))
 (segment (start 102.4925 65.39) (end 104.22 65.39) (width 0.5) (layer "F.Cu") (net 5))
 (segment (start 104.22 62.01) (end 104.21 62) (width 0.5) (layer "F.Cu") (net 5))
 (segment (start 93.8125 73.1125) (end 93.795 73.13) (width 0.5) (layer "F.Cu") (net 7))
 (segment (start 93.8125 70.42) (end 93.8125 73.1125) (width 0.5) (layer "F.Cu") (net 7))
 (segment (start 96.02 73.13) (end 93.795 73.13) (width 0.5) (layer "F.Cu") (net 7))
 (segment (start 96.8175 72.3325) (end 96.02 73.13) (width 0.5) (layer "F.Cu") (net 7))
 (segment (start 96.8175 71.42) (end 96.8175 72.3325) (width 0.5) (layer "F.Cu") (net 7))
 (segment (start 97.89 69.2875) (end 97.89 74.075) (width 0.5) (layer "F.Cu") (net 1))
 (segment (start 97.89 74.075) (end 97.895 74.08) (width 0.5) (layer "F.Cu") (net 1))
 (segment (start 97.895 74.08) (end 100.6275 74.08) (width 0.5) (layer "F.Cu") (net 1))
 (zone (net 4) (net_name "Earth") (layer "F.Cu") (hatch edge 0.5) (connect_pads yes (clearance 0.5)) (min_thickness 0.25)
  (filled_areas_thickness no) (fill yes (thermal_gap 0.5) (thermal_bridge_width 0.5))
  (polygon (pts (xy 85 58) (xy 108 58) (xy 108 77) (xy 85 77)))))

